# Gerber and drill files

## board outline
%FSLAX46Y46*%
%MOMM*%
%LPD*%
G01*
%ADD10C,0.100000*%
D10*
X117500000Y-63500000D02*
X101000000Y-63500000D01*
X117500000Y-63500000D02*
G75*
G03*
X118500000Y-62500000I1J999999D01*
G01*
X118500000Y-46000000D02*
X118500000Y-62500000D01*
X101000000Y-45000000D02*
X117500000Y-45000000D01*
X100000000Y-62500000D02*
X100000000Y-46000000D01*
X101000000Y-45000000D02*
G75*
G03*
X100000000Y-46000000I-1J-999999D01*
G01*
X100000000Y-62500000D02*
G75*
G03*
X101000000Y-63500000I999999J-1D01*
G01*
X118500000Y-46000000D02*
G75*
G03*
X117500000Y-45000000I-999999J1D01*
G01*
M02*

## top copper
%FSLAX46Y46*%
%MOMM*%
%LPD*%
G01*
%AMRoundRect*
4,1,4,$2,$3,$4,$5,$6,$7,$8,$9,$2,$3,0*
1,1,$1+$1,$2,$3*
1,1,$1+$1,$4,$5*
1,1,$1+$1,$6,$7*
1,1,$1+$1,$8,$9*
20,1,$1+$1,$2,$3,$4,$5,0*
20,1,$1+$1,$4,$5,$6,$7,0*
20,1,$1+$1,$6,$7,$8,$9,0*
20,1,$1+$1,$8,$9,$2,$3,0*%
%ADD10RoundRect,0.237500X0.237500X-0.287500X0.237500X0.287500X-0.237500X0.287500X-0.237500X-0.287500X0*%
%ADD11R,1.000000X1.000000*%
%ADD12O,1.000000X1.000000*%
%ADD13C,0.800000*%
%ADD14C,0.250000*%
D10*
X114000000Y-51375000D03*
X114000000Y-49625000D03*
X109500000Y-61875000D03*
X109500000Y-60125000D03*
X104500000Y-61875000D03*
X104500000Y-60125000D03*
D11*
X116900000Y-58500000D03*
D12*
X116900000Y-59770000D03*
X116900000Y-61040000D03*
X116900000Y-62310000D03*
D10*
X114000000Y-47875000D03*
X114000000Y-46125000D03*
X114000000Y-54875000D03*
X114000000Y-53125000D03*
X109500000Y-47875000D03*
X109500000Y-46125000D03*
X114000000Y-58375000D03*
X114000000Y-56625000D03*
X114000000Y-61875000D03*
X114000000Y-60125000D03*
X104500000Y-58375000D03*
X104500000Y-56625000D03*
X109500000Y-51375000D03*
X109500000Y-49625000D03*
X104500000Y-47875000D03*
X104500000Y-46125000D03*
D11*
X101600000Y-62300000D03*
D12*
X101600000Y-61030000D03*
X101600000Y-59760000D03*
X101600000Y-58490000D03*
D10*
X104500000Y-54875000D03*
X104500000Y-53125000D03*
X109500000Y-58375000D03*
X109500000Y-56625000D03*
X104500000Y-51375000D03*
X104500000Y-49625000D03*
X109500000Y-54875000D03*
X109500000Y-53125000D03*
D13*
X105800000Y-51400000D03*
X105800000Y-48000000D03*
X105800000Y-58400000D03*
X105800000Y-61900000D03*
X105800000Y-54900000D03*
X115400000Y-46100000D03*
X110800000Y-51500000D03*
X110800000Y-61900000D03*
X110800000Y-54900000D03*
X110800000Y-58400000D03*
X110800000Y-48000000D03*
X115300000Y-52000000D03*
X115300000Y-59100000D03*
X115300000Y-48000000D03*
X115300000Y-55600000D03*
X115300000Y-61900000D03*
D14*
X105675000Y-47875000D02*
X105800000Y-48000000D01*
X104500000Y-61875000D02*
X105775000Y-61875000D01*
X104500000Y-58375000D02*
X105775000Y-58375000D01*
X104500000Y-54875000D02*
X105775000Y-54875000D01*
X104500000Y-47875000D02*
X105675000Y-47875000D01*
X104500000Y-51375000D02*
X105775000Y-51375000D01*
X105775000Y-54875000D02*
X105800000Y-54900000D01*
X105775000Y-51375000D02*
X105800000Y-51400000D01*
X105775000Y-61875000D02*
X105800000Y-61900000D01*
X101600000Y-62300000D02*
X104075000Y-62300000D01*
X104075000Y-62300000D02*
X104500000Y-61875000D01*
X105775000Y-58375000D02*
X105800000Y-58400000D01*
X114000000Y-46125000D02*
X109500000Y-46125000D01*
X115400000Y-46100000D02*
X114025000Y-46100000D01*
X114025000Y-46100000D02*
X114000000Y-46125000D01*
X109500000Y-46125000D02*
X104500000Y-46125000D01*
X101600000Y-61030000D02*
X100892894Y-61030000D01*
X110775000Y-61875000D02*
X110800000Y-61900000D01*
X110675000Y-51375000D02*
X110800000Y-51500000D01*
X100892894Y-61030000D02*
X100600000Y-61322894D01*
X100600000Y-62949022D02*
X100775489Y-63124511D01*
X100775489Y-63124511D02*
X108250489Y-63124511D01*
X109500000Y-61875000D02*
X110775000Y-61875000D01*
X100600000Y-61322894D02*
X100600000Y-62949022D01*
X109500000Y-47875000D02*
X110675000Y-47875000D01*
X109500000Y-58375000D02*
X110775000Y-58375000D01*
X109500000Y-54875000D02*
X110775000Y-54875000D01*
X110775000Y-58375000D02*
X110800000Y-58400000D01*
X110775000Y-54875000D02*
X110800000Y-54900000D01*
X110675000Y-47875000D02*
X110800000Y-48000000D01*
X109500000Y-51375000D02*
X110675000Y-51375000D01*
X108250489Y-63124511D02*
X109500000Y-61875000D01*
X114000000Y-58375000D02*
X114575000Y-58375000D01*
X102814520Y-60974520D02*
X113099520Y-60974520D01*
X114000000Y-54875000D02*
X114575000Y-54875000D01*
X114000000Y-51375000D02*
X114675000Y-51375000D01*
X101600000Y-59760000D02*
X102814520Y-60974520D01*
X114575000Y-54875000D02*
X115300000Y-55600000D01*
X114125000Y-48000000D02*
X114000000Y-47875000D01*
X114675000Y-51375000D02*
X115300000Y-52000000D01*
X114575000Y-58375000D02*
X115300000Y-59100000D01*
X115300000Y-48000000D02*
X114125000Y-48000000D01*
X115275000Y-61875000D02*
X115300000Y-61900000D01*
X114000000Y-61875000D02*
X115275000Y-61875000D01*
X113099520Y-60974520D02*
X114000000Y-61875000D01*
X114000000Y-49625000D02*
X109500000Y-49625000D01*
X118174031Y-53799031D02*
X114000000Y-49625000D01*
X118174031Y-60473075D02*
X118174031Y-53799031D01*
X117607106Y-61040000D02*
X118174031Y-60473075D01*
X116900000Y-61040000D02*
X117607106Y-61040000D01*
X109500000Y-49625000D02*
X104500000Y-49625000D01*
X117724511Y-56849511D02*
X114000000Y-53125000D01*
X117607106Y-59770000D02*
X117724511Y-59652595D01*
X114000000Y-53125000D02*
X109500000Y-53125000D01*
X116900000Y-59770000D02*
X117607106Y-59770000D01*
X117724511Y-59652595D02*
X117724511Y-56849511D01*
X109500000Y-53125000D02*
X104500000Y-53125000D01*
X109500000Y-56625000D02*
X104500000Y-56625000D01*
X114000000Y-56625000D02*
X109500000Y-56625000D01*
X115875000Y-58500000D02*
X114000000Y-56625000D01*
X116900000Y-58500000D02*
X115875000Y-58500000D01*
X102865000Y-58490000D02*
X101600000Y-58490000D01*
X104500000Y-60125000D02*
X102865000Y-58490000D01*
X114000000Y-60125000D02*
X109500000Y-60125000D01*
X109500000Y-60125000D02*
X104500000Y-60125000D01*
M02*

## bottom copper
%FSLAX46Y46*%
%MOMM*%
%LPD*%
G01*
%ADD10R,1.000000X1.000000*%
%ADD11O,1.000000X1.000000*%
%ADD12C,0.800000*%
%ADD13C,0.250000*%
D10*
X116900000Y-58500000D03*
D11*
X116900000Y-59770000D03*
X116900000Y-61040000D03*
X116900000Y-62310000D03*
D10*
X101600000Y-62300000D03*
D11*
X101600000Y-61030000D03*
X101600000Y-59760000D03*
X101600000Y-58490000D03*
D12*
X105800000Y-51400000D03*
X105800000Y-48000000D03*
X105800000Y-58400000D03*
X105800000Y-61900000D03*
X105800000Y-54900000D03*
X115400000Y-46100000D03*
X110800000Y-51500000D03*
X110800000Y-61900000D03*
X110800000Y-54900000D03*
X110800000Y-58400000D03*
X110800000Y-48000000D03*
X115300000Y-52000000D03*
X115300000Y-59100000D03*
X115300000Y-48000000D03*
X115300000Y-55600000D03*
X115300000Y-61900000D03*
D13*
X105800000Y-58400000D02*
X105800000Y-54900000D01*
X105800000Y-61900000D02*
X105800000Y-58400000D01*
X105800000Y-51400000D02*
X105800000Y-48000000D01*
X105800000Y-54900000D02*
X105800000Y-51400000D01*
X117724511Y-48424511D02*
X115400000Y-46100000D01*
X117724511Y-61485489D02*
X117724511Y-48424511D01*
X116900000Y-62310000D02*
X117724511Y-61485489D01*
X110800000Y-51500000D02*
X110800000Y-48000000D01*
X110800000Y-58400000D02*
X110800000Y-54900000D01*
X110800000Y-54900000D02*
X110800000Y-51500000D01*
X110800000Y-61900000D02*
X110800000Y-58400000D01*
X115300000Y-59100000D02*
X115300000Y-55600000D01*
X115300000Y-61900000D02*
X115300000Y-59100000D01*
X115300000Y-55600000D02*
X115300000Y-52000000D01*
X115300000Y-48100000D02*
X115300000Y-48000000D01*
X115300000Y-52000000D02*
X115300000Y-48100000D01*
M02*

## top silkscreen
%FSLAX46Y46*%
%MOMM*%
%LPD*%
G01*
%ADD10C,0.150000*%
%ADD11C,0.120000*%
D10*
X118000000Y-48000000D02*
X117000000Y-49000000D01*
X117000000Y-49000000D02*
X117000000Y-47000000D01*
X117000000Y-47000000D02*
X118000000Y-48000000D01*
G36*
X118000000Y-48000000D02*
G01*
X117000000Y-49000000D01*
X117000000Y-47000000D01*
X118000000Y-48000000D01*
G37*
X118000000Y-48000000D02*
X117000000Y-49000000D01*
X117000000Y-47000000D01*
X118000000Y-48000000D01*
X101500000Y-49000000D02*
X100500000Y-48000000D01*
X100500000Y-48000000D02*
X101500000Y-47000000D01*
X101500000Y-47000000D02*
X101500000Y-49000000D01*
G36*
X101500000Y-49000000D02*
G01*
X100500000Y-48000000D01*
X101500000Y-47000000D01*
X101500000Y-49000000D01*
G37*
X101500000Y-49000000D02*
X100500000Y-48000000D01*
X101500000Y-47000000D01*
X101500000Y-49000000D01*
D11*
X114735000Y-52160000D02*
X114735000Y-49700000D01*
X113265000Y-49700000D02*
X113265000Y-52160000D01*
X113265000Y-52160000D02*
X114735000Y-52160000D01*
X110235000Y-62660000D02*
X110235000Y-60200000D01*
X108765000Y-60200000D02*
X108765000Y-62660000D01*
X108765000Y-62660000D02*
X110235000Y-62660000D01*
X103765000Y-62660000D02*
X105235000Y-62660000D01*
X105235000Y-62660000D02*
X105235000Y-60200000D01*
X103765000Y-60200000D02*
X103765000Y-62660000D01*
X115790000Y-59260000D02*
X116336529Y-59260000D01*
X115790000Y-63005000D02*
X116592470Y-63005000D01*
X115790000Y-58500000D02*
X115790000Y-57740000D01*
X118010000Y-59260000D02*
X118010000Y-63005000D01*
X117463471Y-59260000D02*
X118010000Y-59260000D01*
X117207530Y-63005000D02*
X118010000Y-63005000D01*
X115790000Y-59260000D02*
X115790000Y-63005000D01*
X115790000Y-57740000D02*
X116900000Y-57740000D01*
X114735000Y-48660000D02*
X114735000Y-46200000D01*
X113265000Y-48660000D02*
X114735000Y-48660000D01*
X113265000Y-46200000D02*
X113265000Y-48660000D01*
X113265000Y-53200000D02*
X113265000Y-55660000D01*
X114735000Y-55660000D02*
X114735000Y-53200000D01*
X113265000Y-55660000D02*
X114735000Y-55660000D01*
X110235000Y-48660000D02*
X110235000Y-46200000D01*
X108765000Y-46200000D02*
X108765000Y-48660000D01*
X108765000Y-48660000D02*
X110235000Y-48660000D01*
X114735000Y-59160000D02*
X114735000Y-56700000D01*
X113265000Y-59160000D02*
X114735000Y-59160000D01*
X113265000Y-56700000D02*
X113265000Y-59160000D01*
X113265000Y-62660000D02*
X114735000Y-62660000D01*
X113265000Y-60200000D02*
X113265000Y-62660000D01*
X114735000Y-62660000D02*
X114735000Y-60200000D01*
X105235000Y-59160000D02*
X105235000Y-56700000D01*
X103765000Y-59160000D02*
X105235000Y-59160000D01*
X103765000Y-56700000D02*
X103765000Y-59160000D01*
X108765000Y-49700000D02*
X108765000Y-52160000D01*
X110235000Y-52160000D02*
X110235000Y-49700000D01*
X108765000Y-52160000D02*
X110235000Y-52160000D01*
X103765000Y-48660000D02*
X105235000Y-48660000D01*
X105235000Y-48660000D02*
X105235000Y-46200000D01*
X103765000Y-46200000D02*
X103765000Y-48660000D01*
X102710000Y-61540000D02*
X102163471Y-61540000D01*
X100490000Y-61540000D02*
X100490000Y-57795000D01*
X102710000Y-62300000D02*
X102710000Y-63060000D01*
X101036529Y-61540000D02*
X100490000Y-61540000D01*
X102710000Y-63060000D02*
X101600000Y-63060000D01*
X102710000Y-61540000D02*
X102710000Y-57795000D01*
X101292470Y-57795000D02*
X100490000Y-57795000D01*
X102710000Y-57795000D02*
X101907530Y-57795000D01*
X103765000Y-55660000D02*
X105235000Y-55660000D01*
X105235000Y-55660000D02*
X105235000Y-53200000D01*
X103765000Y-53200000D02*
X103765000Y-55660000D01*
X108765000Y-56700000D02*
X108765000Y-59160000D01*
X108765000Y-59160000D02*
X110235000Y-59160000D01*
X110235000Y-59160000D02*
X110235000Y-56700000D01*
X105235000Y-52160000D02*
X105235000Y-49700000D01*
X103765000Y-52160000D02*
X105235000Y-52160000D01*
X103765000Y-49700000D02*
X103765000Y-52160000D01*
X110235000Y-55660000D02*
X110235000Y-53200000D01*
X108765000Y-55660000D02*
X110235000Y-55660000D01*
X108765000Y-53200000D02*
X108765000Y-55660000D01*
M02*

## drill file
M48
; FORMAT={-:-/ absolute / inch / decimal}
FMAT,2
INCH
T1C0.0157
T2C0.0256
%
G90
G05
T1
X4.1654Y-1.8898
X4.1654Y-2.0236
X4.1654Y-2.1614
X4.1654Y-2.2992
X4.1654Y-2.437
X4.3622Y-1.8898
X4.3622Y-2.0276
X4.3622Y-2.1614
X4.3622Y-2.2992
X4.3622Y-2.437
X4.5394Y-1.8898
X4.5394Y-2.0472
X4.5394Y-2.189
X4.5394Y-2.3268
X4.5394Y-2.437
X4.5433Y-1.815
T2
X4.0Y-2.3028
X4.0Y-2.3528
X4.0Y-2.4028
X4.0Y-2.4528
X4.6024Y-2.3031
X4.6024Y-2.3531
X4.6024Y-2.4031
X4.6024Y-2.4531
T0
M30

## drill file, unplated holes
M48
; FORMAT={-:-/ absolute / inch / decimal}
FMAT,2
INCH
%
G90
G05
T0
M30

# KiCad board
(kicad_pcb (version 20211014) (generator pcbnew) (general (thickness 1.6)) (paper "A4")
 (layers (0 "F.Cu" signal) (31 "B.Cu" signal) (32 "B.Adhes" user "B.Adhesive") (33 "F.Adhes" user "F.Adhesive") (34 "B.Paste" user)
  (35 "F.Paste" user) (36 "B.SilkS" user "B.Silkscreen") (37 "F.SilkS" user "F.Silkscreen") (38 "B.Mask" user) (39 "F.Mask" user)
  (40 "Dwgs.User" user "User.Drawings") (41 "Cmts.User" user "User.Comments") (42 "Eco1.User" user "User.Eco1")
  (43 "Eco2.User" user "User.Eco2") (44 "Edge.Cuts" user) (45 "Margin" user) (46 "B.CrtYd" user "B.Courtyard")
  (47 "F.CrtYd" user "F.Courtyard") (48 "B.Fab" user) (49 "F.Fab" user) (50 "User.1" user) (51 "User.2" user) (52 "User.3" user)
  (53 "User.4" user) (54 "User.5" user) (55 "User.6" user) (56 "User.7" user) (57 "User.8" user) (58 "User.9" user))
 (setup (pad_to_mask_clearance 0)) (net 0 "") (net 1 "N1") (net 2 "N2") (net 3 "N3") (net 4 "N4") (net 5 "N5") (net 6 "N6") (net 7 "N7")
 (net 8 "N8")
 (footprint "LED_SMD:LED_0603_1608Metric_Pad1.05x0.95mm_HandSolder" (layer "F.Cu") (at 114 50.5 90)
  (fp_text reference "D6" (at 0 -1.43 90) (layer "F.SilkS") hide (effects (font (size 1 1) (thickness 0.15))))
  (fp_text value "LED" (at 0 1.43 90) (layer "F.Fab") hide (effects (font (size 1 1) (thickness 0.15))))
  (fp_line (start -1.66 0.735) (end 0.8 0.735) (layer "F.SilkS") (width 0.12))
  (fp_line (start 0.8 -0.735) (end -1.66 -0.735) (layer "F.SilkS") (width 0.12))
  (fp_line (start -1.66 -0.735) (end -1.66 0.735) (layer "F.SilkS") (width 0.12))
  (pad "1" smd roundrect locked (at -0.875 0 90) (size 1.05 0.95) (layers "F.Cu" "F.Paste" "F.Mask") (roundrect_rratio 0.25) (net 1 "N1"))
  (pad "2" smd roundrect locked (at 0.875 0 90) (size 1.05 0.95) (layers "F.Cu" "F.Paste" "F.Mask") (roundrect_rratio 0.25) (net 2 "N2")))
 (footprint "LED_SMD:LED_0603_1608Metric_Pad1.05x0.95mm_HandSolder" (layer "F.Cu") (at 109.5 61 90)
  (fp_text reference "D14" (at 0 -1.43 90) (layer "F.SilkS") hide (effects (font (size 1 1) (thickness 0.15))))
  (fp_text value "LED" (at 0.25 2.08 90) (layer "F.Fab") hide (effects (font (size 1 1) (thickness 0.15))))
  (fp_line (start -1.66 0.735) (end 0.8 0.735) (layer "F.SilkS") (width 0.12))
  (fp_line (start 0.8 -0.735) (end -1.66 -0.735) (layer "F.SilkS") (width 0.12))
  (fp_line (start -1.66 -0.735) (end -1.66 0.735) (layer "F.SilkS") (width 0.12))
  (pad "1" smd roundrect locked (at -0.875 0 90) (size 1.05 0.95) (layers "F.Cu" "F.Paste" "F.Mask") (roundrect_rratio 0.25) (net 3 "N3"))
  (pad "2" smd roundrect locked (at 0.875 0 90) (size 1.05 0.95) (layers "F.Cu" "F.Paste" "F.Mask") (roundrect_rratio 0.25) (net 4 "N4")))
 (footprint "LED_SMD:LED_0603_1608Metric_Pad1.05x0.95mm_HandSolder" (layer "F.Cu") (at 104.5 61 90)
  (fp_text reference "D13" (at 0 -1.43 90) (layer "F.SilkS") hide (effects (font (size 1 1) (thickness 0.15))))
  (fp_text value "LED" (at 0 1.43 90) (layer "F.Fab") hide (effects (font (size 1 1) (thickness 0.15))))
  (fp_line (start -1.66 -0.735) (end -1.66 0.735) (layer "F.SilkS") (width 0.12))
  (fp_line (start -1.66 0.735) (end 0.8 0.735) (layer "F.SilkS") (width 0.12))
  (fp_line (start 0.8 -0.735) (end -1.66 -0.735) (layer "F.SilkS") (width 0.12))
  (pad "1" smd roundrect locked (at -0.875 0 90) (size 1.05 0.95) (layers "F.Cu" "F.Paste" "F.Mask") (roundrect_rratio 0.25) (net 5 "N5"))
  (pad "2" smd roundrect locked (at 0.875 0 90) (size 1.05 0.95) (layers "F.Cu" "F.Paste" "F.Mask") (roundrect_rratio 0.25) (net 4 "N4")))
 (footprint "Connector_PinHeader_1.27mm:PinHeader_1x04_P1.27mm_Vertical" (layer "F.Cu") (at 116.9 58.5)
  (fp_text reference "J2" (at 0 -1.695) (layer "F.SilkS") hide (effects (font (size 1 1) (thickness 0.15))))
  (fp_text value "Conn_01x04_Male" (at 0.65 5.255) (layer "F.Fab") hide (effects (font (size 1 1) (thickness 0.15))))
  (fp_line (start -1.11 0.76) (end -0.563471 0.76) (layer "F.SilkS") (width 0.12))
  (fp_line (start -1.11 4.505) (end -0.30753 4.505) (layer "F.SilkS") (width 0.12))
  (fp_line (start -1.11 0) (end -1.11 -0.76) (layer "F.SilkS") (width 0.12))
  (fp_line (start 1.11 0.76) (end 1.11 4.505) (layer "F.SilkS") (width 0.12))
  (fp_line (start 0.563471 0.76) (end 1.11 0.76) (layer "F.SilkS") (width 0.12))
  (fp_line (start 0.30753 4.505) (end 1.11 4.505) (layer "F.SilkS") (width 0.12))
  (fp_line (start -1.11 0.76) (end -1.11 4.505) (layer "F.SilkS") (width 0.12))
  (fp_line (start -1.11 -0.76) (end 0 -0.76) (layer "F.SilkS") (width 0.12))
  (pad "1" thru_hole rect locked (at 0 0) (size 1 1) (drill 0.65) (layers *.Cu *.Mask) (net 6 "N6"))
  (pad "2" thru_hole oval locked (at 0 1.27) (size 1 1) (drill 0.65) (layers *.Cu *.Mask) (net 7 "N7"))
  (pad "3" thru_hole oval locked (at 0 2.54) (size 1 1) (drill 0.65) (layers *.Cu *.Mask) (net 2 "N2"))
  (pad "4" thru_hole oval locked (at 0 3.81) (size 1 1) (drill 0.65) (layers *.Cu *.Mask) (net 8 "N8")))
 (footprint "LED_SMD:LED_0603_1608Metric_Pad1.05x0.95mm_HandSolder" (layer "F.Cu") (at 114 47 90)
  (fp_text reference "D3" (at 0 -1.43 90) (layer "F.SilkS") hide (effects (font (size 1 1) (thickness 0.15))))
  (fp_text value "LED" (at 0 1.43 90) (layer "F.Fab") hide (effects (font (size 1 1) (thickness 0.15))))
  (fp_line (start -1.66 0.735) (end 0.8 0.735) (layer "F.SilkS") (width 0.12))
  (fp_line (start -1.66 -0.735) (end -1.66 0.735) (layer "F.SilkS") (width 0.12))
  (fp_line (start 0.8 -0.735) (end -1.66 -0.735) (layer "F.SilkS") (width 0.12))
  (pad "1" smd roundrect locked (at -0.875 0 90) (size 1.05 0.95) (layers "F.Cu" "F.Paste" "F.Mask") (roundrect_rratio 0.25) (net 1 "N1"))
  (pad "2" smd roundrect locked (at 0.875 0 90) (size 1.05 0.95) (layers "F.Cu" "F.Paste" "F.Mask") (roundrect_rratio 0.25) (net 8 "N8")))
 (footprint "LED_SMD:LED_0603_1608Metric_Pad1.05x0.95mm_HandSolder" (layer "F.Cu") (at 114 54 90)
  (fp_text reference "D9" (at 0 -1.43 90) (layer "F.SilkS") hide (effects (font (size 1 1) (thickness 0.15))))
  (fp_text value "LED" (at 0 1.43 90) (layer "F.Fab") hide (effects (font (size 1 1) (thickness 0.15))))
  (fp_line (start 0.8 -0.735) (end -1.66 -0.735) (layer "F.SilkS") (width 0.12))
  (fp_line (start -1.66 0.735) (end 0.8 0.735) (layer "F.SilkS") (width 0.12))
  (fp_line (start -1.66 -0.735) (end -1.66 0.735) (layer "F.SilkS") (width 0.12))
  (pad "1" smd roundrect locked (at -0.875 0 90) (size 1.05 0.95) (layers "F.Cu" "F.Paste" "F.Mask") (roundrect_rratio 0.25) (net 1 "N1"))
  (pad "2" smd roundrect locked (at 0.875 0 90) (size 1.05 0.95) (layers "F.Cu" "F.Paste" "F.Mask") (roundrect_rratio 0.25) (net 7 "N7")))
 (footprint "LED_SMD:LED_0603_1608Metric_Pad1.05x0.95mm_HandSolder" (layer "F.Cu") (at 109.5 47 90)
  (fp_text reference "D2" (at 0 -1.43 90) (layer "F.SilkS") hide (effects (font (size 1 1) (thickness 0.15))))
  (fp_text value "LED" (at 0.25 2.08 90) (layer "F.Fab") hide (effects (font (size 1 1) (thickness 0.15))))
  (fp_line (start -1.66 0.735) (end 0.8 0.735) (layer "F.SilkS") (width 0.12))
  (fp_line (start 0.8 -0.735) (end -1.66 -0.735) (layer "F.SilkS") (width 0.12))
  (fp_line (start -1.66 -0.735) (end -1.66 0.735) (layer "F.SilkS") (width 0.12))
  (pad "1" smd roundrect locked (at -0.875 0 90) (size 1.05 0.95) (layers "F.Cu" "F.Paste" "F.Mask") (roundrect_rratio 0.25) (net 3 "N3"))
  (pad "2" smd roundrect locked (at 0.875 0 90) (size 1.05 0.95) (layers "F.Cu" "F.Paste" "F.Mask") (roundrect_rratio 0.25) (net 8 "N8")))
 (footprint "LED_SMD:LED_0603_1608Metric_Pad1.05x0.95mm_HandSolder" (layer "F.Cu") (at 114 57.5 90)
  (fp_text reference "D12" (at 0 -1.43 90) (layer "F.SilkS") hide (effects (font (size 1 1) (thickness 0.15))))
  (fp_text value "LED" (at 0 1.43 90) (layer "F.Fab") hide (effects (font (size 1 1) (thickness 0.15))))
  (fp_line (start -1.66 0.735) (end 0.8 0.735) (layer "F.SilkS") (width 0.12))
  (fp_line (start -1.66 -0.735) (end -1.66 0.735) (layer "F.SilkS") (width 0.12))
  (fp_line (start 0.8 -0.735) (end -1.66 -0.735) (layer "F.SilkS") (width 0.12))
  (pad "1" smd roundrect locked (at -0.875 0 90) (size 1.05 0.95) (layers "F.Cu" "F.Paste" "F.Mask") (roundrect_rratio 0.25) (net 1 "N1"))
  (pad "2" smd roundrect locked (at 0.875 0 90) (size 1.05 0.95) (layers "F.Cu" "F.Paste" "F.Mask") (roundrect_rratio 0.25) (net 6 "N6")))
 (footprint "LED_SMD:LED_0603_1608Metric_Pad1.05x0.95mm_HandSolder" (layer "F.Cu") (at 114 61 90)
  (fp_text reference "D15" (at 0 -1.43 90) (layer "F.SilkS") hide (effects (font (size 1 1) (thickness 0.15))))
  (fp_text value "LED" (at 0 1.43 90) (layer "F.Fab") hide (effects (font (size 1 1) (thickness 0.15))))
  (fp_line (start -1.66 -0.735) (end -1.66 0.735) (layer "F.SilkS") (width 0.12))
  (fp_line (start 0.8 -0.735) (end -1.66 -0.735) (layer "F.SilkS") (width 0.12))
  (fp_line (start -1.66 0.735) (end 0.8 0.735) (layer "F.SilkS") (width 0.12))
  (pad "1" smd roundrect locked (at -0.875 0 90) (size 1.05 0.95) (layers "F.Cu" "F.Paste" "F.Mask") (roundrect_rratio 0.25) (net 1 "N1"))
  (pad "2" smd roundrect locked (at 0.875 0 90) (size 1.05 0.95) (layers "F.Cu" "F.Paste" "F.Mask") (roundrect_rratio 0.25) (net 4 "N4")))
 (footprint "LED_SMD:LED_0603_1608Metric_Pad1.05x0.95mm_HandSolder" (layer "F.Cu") (at 104.5 57.5 90)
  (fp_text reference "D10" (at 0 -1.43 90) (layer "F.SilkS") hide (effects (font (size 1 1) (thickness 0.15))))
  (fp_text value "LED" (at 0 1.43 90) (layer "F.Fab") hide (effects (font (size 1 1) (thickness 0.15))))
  (fp_line (start -1.66 0.735) (end 0.8 0.735) (layer "F.SilkS") (width 0.12))
  (fp_line (start -1.66 -0.735) (end -1.66 0.735) (layer "F.SilkS") (width 0.12))
  (fp_line (start 0.8 -0.735) (end -1.66 -0.735) (layer "F.SilkS") (width 0.12))
  (pad "1" smd roundrect locked (at -0.875 0 90) (size 1.05 0.95) (layers "F.Cu" "F.Paste" "F.Mask") (roundrect_rratio 0.25) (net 5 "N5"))
  (pad "2" smd roundrect locked (at 0.875 0 90) (size 1.05 0.95) (layers "F.Cu" "F.Paste" "F.Mask") (roundrect_rratio 0.25) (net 6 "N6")))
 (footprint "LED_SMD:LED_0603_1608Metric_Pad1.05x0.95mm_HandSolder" (layer "F.Cu") (at 109.5 50.5 90)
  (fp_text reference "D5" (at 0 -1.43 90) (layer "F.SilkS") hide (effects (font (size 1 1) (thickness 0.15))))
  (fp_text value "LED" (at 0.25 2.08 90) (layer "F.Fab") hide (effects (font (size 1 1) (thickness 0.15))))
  (fp_line (start 0.8 -0.735) (end -1.66 -0.735) (layer "F.SilkS") (width 0.12))
  (fp_line (start -1.66 0.735) (end 0.8 0.735) (layer "F.SilkS") (width 0.12))
  (fp_line (start -1.66 -0.735) (end -1.66 0.735) (layer "F.SilkS") (width 0.12))
  (pad "1" smd roundrect locked (at -0.875 0 90) (size 1.05 0.95) (layers "F.Cu" "F.Paste" "F.Mask") (roundrect_rratio 0.25) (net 3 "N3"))
  (pad "2" smd roundrect locked (at 0.875 0 90) (size 1.05 0.95) (layers "F.Cu" "F.Paste" "F.Mask") (roundrect_rratio 0.25) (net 2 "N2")))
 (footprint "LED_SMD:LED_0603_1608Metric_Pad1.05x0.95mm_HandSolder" (layer "F.Cu") (at 104.5 47 90)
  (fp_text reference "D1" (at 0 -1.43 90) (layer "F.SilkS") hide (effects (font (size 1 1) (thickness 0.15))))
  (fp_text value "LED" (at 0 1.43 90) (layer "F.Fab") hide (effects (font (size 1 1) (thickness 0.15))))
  (fp_line (start -1.66 -0.735) (end -1.66 0.735) (layer "F.SilkS") (width 0.12))
  (fp_line (start -1.66 0.735) (end 0.8 0.735) (layer "F.SilkS") (width 0.12))
  (fp_line (start 0.8 -0.735) (end -1.66 -0.735) (layer "F.SilkS") (width 0.12))
  (pad "1" smd roundrect locked (at -0.875 0 90) (size 1.05 0.95) (layers "F.Cu" "F.Paste" "F.Mask") (roundrect_rratio 0.25) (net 5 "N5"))
  (pad "2" smd roundrect locked (at 0.875 0 90) (size 1.05 0.95) (layers "F.Cu" "F.Paste" "F.Mask") (roundrect_rratio 0.25) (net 8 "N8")))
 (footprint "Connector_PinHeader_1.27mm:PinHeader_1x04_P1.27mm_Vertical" (layer "F.Cu") (at 101.6 62.3 180)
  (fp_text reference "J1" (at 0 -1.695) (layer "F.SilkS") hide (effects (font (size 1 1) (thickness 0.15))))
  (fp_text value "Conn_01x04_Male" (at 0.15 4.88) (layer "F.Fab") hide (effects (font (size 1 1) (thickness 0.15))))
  (fp_line (start -1.11 0.76) (end -0.563471 0.76) (layer "F.SilkS") (width 0.12))
  (fp_line (start 1.11 0.76) (end 1.11 4.505) (layer "F.SilkS") (width 0.12))
  (fp_line (start -1.11 0) (end -1.11 -0.76) (layer "F.SilkS") (width 0.12))
  (fp_line (start 0.563471 0.76) (end 1.11 0.76) (layer "F.SilkS") (width 0.12))
  (fp_line (start -1.11 -0.76) (end 0 -0.76) (layer "F.SilkS") (width 0.12))
  (fp_line (start -1.11 0.76) (end -1.11 4.505) (layer "F.SilkS") (width 0.12))
  (fp_line (start 0.30753 4.505) (end 1.11 4.505) (layer "F.SilkS") (width 0.12))
  (fp_line (start -1.11 4.505) (end -0.30753 4.505) (layer "F.SilkS") (width 0.12))
  (pad "1" thru_hole rect locked (at 0 0 180) (size 1 1) (drill 0.65) (layers *.Cu *.Mask) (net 5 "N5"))
  (pad "2" thru_hole oval locked (at 0 1.27 180) (size 1 1) (drill 0.65) (layers *.Cu *.Mask) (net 3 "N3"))
  (pad "3" thru_hole oval locked (at 0 2.54 180) (size 1 1) (drill 0.65) (layers *.Cu *.Mask) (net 1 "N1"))
  (pad "4" thru_hole oval locked (at 0 3.81 180) (size 1 1) (drill 0.65) (layers *.Cu *.Mask) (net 4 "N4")))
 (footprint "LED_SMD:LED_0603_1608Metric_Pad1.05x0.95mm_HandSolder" (layer "F.Cu") (at 104.5 54 90)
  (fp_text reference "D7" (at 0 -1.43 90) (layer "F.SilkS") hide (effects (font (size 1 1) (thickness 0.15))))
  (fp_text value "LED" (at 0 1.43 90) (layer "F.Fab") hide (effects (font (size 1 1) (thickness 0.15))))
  (fp_line (start -1.66 -0.735) (end -1.66 0.735) (layer "F.SilkS") (width 0.12))
  (fp_line (start -1.66 0.735) (end 0.8 0.735) (layer "F.SilkS") (width 0.12))
  (fp_line (start 0.8 -0.735) (end -1.66 -0.735) (layer "F.SilkS") (width 0.12))
  (pad "1" smd roundrect locked (at -0.875 0 90) (size 1.05 0.95) (layers "F.Cu" "F.Paste" "F.Mask") (roundrect_rratio 0.25) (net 5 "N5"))
  (pad "2" smd roundrect locked (at 0.875 0 90) (size 1.05 0.95) (layers "F.Cu" "F.Paste" "F.Mask") (roundrect_rratio 0.25) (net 7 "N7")))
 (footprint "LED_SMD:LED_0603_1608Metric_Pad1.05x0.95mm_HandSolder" (layer "F.Cu") (at 109.5 57.5 90)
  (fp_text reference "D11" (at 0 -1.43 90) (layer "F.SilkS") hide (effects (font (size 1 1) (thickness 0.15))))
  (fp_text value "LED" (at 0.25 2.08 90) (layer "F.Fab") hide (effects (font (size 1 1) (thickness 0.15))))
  (fp_line (start 0.8 -0.735) (end -1.66 -0.735) (layer "F.SilkS") (width 0.12))
  (fp_line (start -1.66 -0.735) (end -1.66 0.735) (layer "F.SilkS") (width 0.12))
  (fp_line (start -1.66 0.735) (end 0.8 0.735) (layer "F.SilkS") (width 0.12))
  (pad "1" smd roundrect locked (at -0.875 0 90) (size 1.05 0.95) (layers "F.Cu" "F.Paste" "F.Mask") (roundrect_rratio 0.25) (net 3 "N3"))
  (pad "2" smd roundrect locked (at 0.875 0 90) (size 1.05 0.95) (layers "F.Cu" "F.Paste" "F.Mask") (roundrect_rratio 0.25) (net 6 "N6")))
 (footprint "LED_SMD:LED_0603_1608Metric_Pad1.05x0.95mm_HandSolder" (layer "F.Cu") (at 104.5 50.5 90)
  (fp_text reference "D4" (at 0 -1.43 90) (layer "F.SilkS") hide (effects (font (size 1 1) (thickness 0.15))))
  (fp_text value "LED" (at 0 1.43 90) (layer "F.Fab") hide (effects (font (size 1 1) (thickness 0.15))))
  (fp_line (start -1.66 0.735) (end 0.8 0.735) (layer "F.SilkS") (width 0.12))
  (fp_line (start -1.66 -0.735) (end -1.66 0.735) (layer "F.SilkS") (width 0.12))
  (fp_line (start 0.8 -0.735) (end -1.66 -0.735) (layer "F.SilkS") (width 0.12))
  (pad "1" smd roundrect locked (at -0.875 0 90) (size 1.05 0.95) (layers "F.Cu" "F.Paste" "F.Mask") (roundrect_rratio 0.25) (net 5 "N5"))
  (pad "2" smd roundrect locked (at 0.875 0 90) (size 1.05 0.95) (layers "F.Cu" "F.Paste" "F.Mask") (roundrect_rratio 0.25) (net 2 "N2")))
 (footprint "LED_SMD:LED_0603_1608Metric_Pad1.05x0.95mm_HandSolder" (layer "F.Cu") (at 109.5 54 90)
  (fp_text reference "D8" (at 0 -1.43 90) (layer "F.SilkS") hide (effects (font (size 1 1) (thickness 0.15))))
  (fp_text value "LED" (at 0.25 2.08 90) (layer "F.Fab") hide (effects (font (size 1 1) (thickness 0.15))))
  (fp_line (start -1.66 0.735) (end 0.8 0.735) (layer "F.SilkS") (width 0.12))
  (fp_line (start -1.66 -0.735) (end -1.66 0.735) (layer "F.SilkS") (width 0.12))
  (fp_line (start 0.8 -0.735) (end -1.66 -0.735) (layer "F.SilkS") (width 0.12))
  (pad "1" smd roundrect locked (at -0.875 0 90) (size 1.05 0.95) (layers "F.Cu" "F.Paste" "F.Mask") (roundrect_rratio 0.25) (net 3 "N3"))
  (pad "2" smd roundrect locked (at 0.875 0 90) (size 1.05 0.95) (layers "F.Cu" "F.Paste" "F.Mask") (roundrect_rratio 0.25) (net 7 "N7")))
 (gr_poly (pts (xy 118 48) (xy 117 49) (xy 117 47)) (layer "F.SilkS") (width 0.15) (fill solid))
 (gr_poly (pts (xy 101.5 49) (xy 100.5 48) (xy 101.5 47)) (layer "F.SilkS") (width 0.15) (fill solid))
 (gr_line (start 117.5 63.5) (end 101 63.5) (layer "Edge.Cuts") (width 0.1))
 (gr_arc (start 118.5 62.5) (mid 118.207107 63.207107) (end 117.5 63.5) (layer "Edge.Cuts") (width 0.1))
 (gr_line (start 118.5 46) (end 118.5 62.5) (layer "Edge.Cuts") (width 0.1))
 (gr_line (start 101 45) (end 117.5 45) (layer "Edge.Cuts") (width 0.1))
 (gr_line (start 100 62.5) (end 100 46) (layer "Edge.Cuts") (width 0.1))
 (gr_arc (start 100 46) (mid 100.292893 45.292893) (end 101 45) (layer "Edge.Cuts") (width 0.1))
 (gr_arc (start 101 63.5) (mid 100.292893 63.207107) (end 100 62.5) (layer "Edge.Cuts") (width 0.1))
 (gr_arc (start 117.5 45) (mid 118.207107 45.292893) (end 118.5 46) (layer "Edge.Cuts") (width 0.1))
 (segment (start 105.675 47.875) (end 105.8 48) (width 0.25) (layer "F.Cu") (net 5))
 (segment (start 104.5 61.875) (end 105.775 61.875) (width 0.25) (layer "F.Cu") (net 5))
 (segment (start 104.5 58.375) (end 105.775 58.375) (width 0.25) (layer "F.Cu") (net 5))
 (segment (start 104.5 54.875) (end 105.775 54.875) (width 0.25) (layer "F.Cu") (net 5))
 (segment (start 104.5 47.875) (end 105.675 47.875) (width 0.25) (layer "F.Cu") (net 5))
 (segment (start 104.5 51.375) (end 105.775 51.375) (width 0.25) (layer "F.Cu") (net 5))
 (segment (start 105.775 54.875) (end 105.8 54.9) (width 0.25) (layer "F.Cu") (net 5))
 (segment (start 105.775 51.375) (end 105.8 51.4) (width 0.25) (layer "F.Cu") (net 5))
 (segment (start 105.775 61.875) (end 105.8 61.9) (width 0.25) (layer "F.Cu") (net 5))
 (segment (start 101.6 62.3) (end 104.075 62.3) (width 0.25) (layer "F.Cu") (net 5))
 (segment (start 104.075 62.3) (end 104.5 61.875) (width 0.25) (layer "F.Cu") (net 5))
 (segment (start 105.775 58.375) (end 105.8 58.4) (width 0.25) (layer "F.Cu") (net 5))
 (via (at 105.8 51.4) (size 0.8) (drill 0.4) (layers "F.Cu" "B.Cu") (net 5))
 (via (at 105.8 48) (size 0.8) (drill 0.4) (layers "F.Cu" "B.Cu") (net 5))
 (via (at 105.8 58.4) (size 0.8) (drill 0.4) (layers "F.Cu" "B.Cu") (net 5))
 (via (at 105.8 61.9) (size 0.8) (drill 0.4) (layers "F.Cu" "B.Cu") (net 5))
 (via (at 105.8 54.9) (size 0.8) (drill 0.4) (layers "F.Cu" "B.Cu") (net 5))
 (segment (start 105.8 58.4) (end 105.8 54.9) (width 0.25) (layer "B.Cu") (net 5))
 (segment (start 105.8 61.9) (end 105.8 58.4) (width 0.25) (layer "B.Cu") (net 5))
 (segment (start 105.8 51.4) (end 105.8 48) (width 0.25) (layer "B.Cu") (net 5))
 (segment (start 105.8 54.9) (end 105.8 51.4) (width 0.25) (layer "B.Cu") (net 5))
 (segment (start 114 46.125) (end 109.5 46.125) (width 0.25) (layer "F.Cu") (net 8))
 (segment (start 115.4 46.1) (end 114.025 46.1) (width 0.25) (layer "F.Cu") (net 8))
 (segment (start 114.025 46.1) (end 114 46.125) (width 0.25) (layer "F.Cu") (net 8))
 (segment (start 109.5 46.125) (end 104.5 46.125) (width 0.25) (layer "F.Cu") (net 8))
 (via (at 115.4 46.1) (size 0.8) (drill 0.4) (layers "F.Cu" "B.Cu") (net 8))
 (segment (start 117.724511 48.424511) (end 115.4 46.1) (width 0.25) (layer "B.Cu") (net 8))
 (segment (start 117.724511 61.485489) (end 117.724511 48.424511) (width 0.25) (layer "B.Cu") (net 8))
 (segment (start 116.9 62.31) (end 117.724511 61.485489) (width 0.25) (layer "B.Cu") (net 8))
 (segment (start 101.6 61.03) (end 100.892894 61.03) (width 0.25) (layer "F.Cu") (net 3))
 (segment (start 110.775 61.875) (end 110.8 61.9) (width 0.25) (layer "F.Cu") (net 3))
 (segment (start 110.675 51.375) (end 110.8 51.5) (width 0.25) (layer "F.Cu") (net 3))
 (segment (start 100.892894 61.03) (end 100.6 61.322894) (width 0.25) (layer "F.Cu") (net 3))
 (segment (start 100.6 62.949022) (end 100.775489 63.124511) (width 0.25) (layer "F.Cu") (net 3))
 (segment (start 100.775489 63.124511) (end 108.250489 63.124511) (width 0.25) (layer "F.Cu") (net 3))
 (segment (start 109.5 61.875) (end 110.775 61.875) (width 0.25) (layer "F.Cu") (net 3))
 (segment (start 100.6 61.322894) (end 100.6 62.949022) (width 0.25) (layer "F.Cu") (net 3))
 (segment (start 109.5 47.875) (end 110.675 47.875) (width 0.25) (layer "F.Cu") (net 3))
 (segment (start 109.5 58.375) (end 110.775 58.375) (width 0.25) (layer "F.Cu") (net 3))
 (segment (start 109.5 54.875) (end 110.775 54.875) (width 0.25) (layer "F.Cu") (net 3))
 (segment (start 110.775 58.375) (end 110.8 58.4) (width 0.25) (layer "F.Cu") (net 3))
 (segment (start 110.775 54.875) (end 110.8 54.9) (width 0.25) (layer "F.Cu") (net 3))
 (segment (start 110.675 47.875) (end 110.8 48) (width 0.25) (layer "F.Cu") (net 3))
 (segment (start 109.5 51.375) (end 110.675 51.375) (width 0.25) (layer "F.Cu") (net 3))
 (segment (start 108.250489 63.124511) (end 109.5 61.875) (width 0.25) (layer "F.Cu") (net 3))
 (via (at 110.8 51.5) (size 0.8) (drill 0.4) (layers "F.Cu" "B.Cu") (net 3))
 (via (at 110.8 61.9) (size 0.8) (drill 0.4) (layers "F.Cu" "B.Cu") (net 3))
 (via (at 110.8 54.9) (size 0.8) (drill 0.4) (layers "F.Cu" "B.Cu") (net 3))
 (via (at 110.8 58.4) (size 0.8) (drill 0.4) (layers "F.Cu" "B.Cu") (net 3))
 (via (at 110.8 48) (size 0.8) (drill 0.4) (layers "F.Cu" "B.Cu") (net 3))
 (segment (start 110.8 51.5) (end 110.8 48) (width 0.25) (layer "B.Cu") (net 3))
 (segment (start 110.8 58.4) (end 110.8 54.9) (width 0.25) (layer "B.Cu") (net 3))
 (segment (start 110.8 54.9) (end 110.8 51.5) (width 0.25) (layer "B.Cu") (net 3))
 (segment (start 110.8 61.9) (end 110.8 58.4) (width 0.25) (layer "B.Cu") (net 3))
 (segment (start 114 58.375) (end 114.575 58.375) (width 0.25) (layer "F.Cu") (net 1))
 (segment (start 102.81452 60.97452) (end 113.09952 60.97452) (width 0.25) (layer "F.Cu") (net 1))
 (segment (start 114 54.875) (end 114.575 54.875) (width 0.25) (layer "F.Cu") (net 1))
 (segment (start 114 51.375) (end 114.675 51.375) (width 0.25) (layer "F.Cu") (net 1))
 (segment (start 101.6 59.76) (end 102.81452 60.97452) (width 0.25) (layer "F.Cu") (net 1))
 (segment (start 114.575 54.875) (end 115.3 55.6) (width 0.25) (layer "F.Cu") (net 1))
 (segment (start 114.125 48) (end 114 47.875) (width 0.25) (layer "F.Cu") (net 1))
 (segment (start 114.675 51.375) (end 115.3 52) (width 0.25) (layer "F.Cu") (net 1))
 (segment (start 114.575 58.375) (end 115.3 59.1) (width 0.25) (layer "F.Cu") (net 1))
 (segment (start 115.3 48) (end 114.125 48) (width 0.25) (layer "F.Cu") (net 1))
 (segment (start 115.275 61.875) (end 115.3 61.9) (width 0.25) (layer "F.Cu") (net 1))
 (segment (start 114 61.875) (end 115.275 61.875) (width 0.25) (layer "F.Cu") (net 1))
 (segment (start 113.09952 60.97452) (end 114 61.875) (width 0.25) (layer "F.Cu") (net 1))
 (via (at 115.3 52) (size 0.8) (drill 0.4) (layers "F.Cu" "B.Cu") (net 1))
 (via (at 115.3 59.1) (size 0.8) (drill 0.4) (layers "F.Cu" "B.Cu") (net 1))
 (via (at 115.3 48) (size 0.8) (drill 0.4) (layers "F.Cu" "B.Cu") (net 1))
 (via (at 115.3 55.6) (size 0.8) (drill 0.4) (layers "F.Cu" "B.Cu") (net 1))
 (via (at 115.3 61.9) (size 0.8) (drill 0.4) (layers "F.Cu" "B.Cu") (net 1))
 (segment (start 115.3 59.1) (end 115.3 55.6) (width 0.25) (layer "B.Cu") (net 1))
 (segment (start 115.3 61.9) (end 115.3 59.1) (width 0.25) (layer "B.Cu") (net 1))
 (segment (start 115.3 55.6) (end 115.3 52) (width 0.25) (layer "B.Cu") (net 1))
 (segment (start 115.3 48.1) (end 115.3 48) (width 0.25) (layer "B.Cu") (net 1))
 (segment (start 115.3 52) (end 115.3 48.1) (width 0.25) (layer "B.Cu") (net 1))
 (segment (start 114 49.625) (end 109.5 49.625) (width 0.25) (layer "F.Cu") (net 2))
 (segment (start 118.174031 53.799031) (end 114 49.625) (width 0.25) (layer "F.Cu") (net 2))
 (segment (start 118.174031 60.473075) (end 118.174031 53.799031) (width 0.25) (layer "F.Cu") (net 2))
 (segment (start 117.607106 61.04) (end 118.174031 60.473075) (width 0.25) (layer "F.Cu") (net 2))
 (segment (start 116.9 61.04) (end 117.607106 61.04) (width 0.25) (layer "F.Cu") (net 2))
 (segment (start 109.5 49.625) (end 104.5 49.625) (width 0.25) (layer "F.Cu") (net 2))
 (segment (start 117.724511 56.849511) (end 114 53.125) (width 0.25) (layer "F.Cu") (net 7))
 (segment (start 117.607106 59.77) (end 117.724511 59.652595) (width 0.25) (layer "F.Cu") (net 7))
 (segment (start 114 53.125) (end 109.5 53.125) (width 0.25) (layer "F.Cu") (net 7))
 (segment (start 116.9 59.77) (end 117.607106 59.77) (width 0.25) (layer "F.Cu") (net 7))
 (segment (start 117.724511 59.652595) (end 117.724511 56.849511) (width 0.25) (layer "F.Cu") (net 7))
 (segment (start 109.5 53.125) (end 104.5 53.125) (width 0.25) (layer "F.Cu") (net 7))
 (segment (start 109.5 56.625) (end 104.5 56.625) (width 0.25) (layer "F.Cu") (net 6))
 (segment (start 114 56.625) (end 109.5 56.625) (width 0.25) (layer "F.Cu") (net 6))
 (segment (start 115.875 58.5) (end 114 56.625) (width 0.25) (layer "F.Cu") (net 6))
 (segment (start 116.9 58.5) (end 115.875 58.5) (width 0.25) (layer "F.Cu") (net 6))
 (segment (start 102.865 58.49) (end 101.6 58.49) (width 0.25) (layer "F.Cu") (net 4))
 (segment (start 104.5 60.125) (end 102.865 58.49) (width 0.25) (layer "F.Cu") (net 4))
 (segment (start 114 60.125) (end 109.5 60.125) (width 0.25) (layer "F.Cu") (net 4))
 (segment (start 109.5 60.125) (end 104.5 60.125) (width 0.25) (layer "F.Cu") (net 4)))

